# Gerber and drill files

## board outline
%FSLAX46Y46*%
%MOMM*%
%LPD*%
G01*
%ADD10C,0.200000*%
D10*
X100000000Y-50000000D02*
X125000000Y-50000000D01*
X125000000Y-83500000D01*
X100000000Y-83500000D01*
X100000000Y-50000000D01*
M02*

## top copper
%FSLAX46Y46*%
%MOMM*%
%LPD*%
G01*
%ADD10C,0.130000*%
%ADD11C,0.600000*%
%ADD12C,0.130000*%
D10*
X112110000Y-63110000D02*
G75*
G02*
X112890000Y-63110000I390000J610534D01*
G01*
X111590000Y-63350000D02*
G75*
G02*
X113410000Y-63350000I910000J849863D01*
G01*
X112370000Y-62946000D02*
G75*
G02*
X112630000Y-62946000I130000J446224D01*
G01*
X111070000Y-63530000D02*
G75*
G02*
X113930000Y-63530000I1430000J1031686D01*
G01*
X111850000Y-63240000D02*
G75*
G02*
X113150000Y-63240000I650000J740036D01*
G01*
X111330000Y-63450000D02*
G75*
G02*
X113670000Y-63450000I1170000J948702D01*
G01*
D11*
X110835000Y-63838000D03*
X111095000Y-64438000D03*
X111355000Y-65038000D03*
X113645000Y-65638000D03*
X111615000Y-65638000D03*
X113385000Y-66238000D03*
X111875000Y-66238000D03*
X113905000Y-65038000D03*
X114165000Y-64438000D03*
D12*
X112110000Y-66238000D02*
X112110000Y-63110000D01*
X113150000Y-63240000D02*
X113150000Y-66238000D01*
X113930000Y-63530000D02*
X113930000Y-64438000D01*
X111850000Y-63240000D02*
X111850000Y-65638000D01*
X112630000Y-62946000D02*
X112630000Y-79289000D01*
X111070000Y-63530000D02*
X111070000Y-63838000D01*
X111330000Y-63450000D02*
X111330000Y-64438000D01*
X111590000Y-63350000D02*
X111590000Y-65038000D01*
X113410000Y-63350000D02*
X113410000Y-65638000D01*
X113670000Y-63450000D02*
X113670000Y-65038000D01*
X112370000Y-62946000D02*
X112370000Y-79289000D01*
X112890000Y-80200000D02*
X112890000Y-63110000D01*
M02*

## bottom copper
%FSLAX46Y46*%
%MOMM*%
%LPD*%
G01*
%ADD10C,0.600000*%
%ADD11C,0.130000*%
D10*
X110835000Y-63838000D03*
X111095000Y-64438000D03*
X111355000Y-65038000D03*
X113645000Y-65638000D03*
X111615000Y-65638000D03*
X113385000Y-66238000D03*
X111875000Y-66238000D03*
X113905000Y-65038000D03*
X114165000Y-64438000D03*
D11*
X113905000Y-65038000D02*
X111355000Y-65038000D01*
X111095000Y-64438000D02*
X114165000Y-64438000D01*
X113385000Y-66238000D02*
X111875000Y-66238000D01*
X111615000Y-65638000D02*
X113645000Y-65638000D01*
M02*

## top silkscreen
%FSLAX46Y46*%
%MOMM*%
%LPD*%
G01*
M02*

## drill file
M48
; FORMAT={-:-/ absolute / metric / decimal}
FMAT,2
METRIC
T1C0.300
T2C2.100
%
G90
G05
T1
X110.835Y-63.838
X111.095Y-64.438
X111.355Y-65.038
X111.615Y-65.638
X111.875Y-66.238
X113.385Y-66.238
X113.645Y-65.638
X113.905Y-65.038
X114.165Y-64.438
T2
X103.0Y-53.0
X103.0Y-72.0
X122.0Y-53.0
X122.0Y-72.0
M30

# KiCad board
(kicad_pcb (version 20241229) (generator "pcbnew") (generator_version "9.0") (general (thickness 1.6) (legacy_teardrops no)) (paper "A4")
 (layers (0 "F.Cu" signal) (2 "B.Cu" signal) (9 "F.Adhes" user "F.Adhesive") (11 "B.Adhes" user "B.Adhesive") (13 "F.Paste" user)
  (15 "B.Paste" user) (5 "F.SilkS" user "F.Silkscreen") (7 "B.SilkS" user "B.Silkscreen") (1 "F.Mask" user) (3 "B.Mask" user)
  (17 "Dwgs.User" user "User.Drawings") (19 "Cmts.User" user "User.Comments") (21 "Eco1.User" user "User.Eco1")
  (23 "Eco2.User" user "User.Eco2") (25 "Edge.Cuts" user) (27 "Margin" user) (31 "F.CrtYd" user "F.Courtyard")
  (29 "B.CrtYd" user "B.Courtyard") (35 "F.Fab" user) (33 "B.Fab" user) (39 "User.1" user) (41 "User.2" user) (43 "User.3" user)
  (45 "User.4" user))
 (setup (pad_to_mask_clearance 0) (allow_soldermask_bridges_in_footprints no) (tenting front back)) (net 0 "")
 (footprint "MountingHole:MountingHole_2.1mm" (layer "F.Cu") (at 122 53)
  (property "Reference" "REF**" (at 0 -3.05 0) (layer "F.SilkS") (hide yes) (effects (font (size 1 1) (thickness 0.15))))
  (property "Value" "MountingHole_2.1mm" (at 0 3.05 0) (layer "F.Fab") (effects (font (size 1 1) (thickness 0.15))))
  (pad "" np_thru_hole circle (at 0 0) (size 2.1 2.1) (drill 2.1) (layers "*.Cu" "*.Mask")))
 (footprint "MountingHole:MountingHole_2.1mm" (layer "F.Cu") (at 103 53)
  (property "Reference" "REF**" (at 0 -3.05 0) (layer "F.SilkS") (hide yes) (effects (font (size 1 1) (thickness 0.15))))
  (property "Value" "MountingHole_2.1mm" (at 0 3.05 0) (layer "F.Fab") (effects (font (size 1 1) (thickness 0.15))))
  (pad "" np_thru_hole circle (at 0 0) (size 2.1 2.1) (drill 2.1) (layers "*.Cu" "*.Mask")))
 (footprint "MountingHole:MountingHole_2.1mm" (layer "F.Cu") (at 103 72)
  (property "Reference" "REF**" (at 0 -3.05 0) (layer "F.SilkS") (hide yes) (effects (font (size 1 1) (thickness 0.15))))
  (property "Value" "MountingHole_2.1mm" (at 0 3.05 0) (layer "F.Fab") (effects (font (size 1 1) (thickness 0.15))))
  (pad "" np_thru_hole circle (at 0 0) (size 2.1 2.1) (drill 2.1) (layers "*.Cu" "*.Mask")))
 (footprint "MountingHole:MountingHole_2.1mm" (layer "F.Cu") (at 122 72)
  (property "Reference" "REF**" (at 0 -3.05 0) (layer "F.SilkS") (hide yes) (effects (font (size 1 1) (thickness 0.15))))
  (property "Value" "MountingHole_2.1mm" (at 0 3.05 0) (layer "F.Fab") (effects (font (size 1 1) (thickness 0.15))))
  (pad "" np_thru_hole circle (at 0 0) (size 2.1 2.1) (drill 2.1) (layers "*.Cu" "*.Mask")))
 (gr_arc (start 112.11 63.11) (mid 112.5 61.775) (end 112.89 63.11) (stroke (width 0.13) (type solid)) (layer "F.Cu"))
 (gr_arc (start 111.59 63.35) (mid 112.5 61.255) (end 113.41 63.35) (stroke (width 0.13) (type solid)) (layer "F.Cu"))
 (gr_arc (start 112.37 62.946) (mid 112.5 62.035001) (end 112.63 62.946) (stroke (width 0.13) (type solid)) (layer "F.Cu"))
 (gr_arc (start 111.07 63.53) (mid 112.5 60.735) (end 113.93 63.53) (stroke (width 0.13) (type solid)) (layer "F.Cu"))
 (gr_arc (start 111.85 63.24) (mid 112.5 61.515) (end 113.15 63.24) (stroke (width 0.13) (type solid)) (layer "F.Cu"))
 (gr_arc (start 111.33 63.45) (mid 112.5 60.995) (end 113.67 63.45) (stroke (width 0.13) (type solid)) (layer "F.Cu"))
 (gr_rect (start 100 50) (end 125 83.5) (stroke (width 0.2) (type solid)) (fill no) (layer "Edge.Cuts"))
 (segment (start 112.11 66.238) (end 112.11 63.11) (width 0.13) (layer "F.Cu") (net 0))
 (segment (start 113.15 63.24) (end 113.15 66.238) (width 0.13) (layer "F.Cu") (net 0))
 (segment (start 113.93 63.53) (end 113.93 64.438) (width 0.13) (layer "F.Cu") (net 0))
 (segment (start 111.85 63.24) (end 111.85 65.638) (width 0.13) (layer "F.Cu") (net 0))
 (segment (start 112.63 62.946) (end 112.63 79.289) (width 0.13) (layer "F.Cu") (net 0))
 (segment (start 111.07 63.53) (end 111.07 63.838) (width 0.13) (layer "F.Cu") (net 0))
 (segment (start 111.33 63.45) (end 111.33 64.438) (width 0.13) (layer "F.Cu") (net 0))
 (segment (start 111.59 63.35) (end 111.59 65.038) (width 0.13) (layer "F.Cu") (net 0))
 (segment (start 113.41 63.35) (end 113.41 65.638) (width 0.13) (layer "F.Cu") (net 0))
 (segment (start 113.67 63.45) (end 113.67 65.038) (width 0.13) (layer "F.Cu") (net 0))
 (segment (start 112.37 62.946) (end 112.37 79.289) (width 0.13) (layer "F.Cu") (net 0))
 (segment (start 112.89 80.2) (end 112.89 63.11) (width 0.13) (layer "F.Cu") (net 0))
 (via (at 110.835 63.838) (size 0.6) (drill 0.3) (layers "F.Cu" "B.Cu") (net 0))
 (via (at 111.095 64.438) (size 0.6) (drill 0.3) (layers "F.Cu" "B.Cu") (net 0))
 (via (at 111.355 65.038) (size 0.6) (drill 0.3) (layers "F.Cu" "B.Cu") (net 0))
 (via (at 113.645 65.638) (size 0.6) (drill 0.3) (layers "F.Cu" "B.Cu") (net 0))
 (via (at 111.615 65.638) (size 0.6) (drill 0.3) (layers "F.Cu" "B.Cu") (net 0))
 (via (at 113.385 66.238) (size 0.6) (drill 0.3) (layers "F.Cu" "B.Cu") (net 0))
 (via (at 111.875 66.238) (size 0.6) (drill 0.3) (layers "F.Cu" "B.Cu") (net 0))
 (via (at 113.905 65.038) (size 0.6) (drill 0.3) (layers "F.Cu" "B.Cu") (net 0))
 (via (at 114.165 64.438) (size 0.6) (drill 0.3) (layers "F.Cu" "B.Cu") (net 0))
 (segment (start 113.905 65.038) (end 111.355 65.038) (width 0.13) (layer "B.Cu") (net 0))
 (segment (start 111.095 64.438) (end 114.165 64.438) (width 0.13) (layer "B.Cu") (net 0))
 (segment (start 113.385 66.238) (end 111.875 66.238) (width 0.13) (layer "B.Cu") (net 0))
 (segment (start 111.615 65.638) (end 113.645 65.638) (width 0.13) (layer "B.Cu") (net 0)))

